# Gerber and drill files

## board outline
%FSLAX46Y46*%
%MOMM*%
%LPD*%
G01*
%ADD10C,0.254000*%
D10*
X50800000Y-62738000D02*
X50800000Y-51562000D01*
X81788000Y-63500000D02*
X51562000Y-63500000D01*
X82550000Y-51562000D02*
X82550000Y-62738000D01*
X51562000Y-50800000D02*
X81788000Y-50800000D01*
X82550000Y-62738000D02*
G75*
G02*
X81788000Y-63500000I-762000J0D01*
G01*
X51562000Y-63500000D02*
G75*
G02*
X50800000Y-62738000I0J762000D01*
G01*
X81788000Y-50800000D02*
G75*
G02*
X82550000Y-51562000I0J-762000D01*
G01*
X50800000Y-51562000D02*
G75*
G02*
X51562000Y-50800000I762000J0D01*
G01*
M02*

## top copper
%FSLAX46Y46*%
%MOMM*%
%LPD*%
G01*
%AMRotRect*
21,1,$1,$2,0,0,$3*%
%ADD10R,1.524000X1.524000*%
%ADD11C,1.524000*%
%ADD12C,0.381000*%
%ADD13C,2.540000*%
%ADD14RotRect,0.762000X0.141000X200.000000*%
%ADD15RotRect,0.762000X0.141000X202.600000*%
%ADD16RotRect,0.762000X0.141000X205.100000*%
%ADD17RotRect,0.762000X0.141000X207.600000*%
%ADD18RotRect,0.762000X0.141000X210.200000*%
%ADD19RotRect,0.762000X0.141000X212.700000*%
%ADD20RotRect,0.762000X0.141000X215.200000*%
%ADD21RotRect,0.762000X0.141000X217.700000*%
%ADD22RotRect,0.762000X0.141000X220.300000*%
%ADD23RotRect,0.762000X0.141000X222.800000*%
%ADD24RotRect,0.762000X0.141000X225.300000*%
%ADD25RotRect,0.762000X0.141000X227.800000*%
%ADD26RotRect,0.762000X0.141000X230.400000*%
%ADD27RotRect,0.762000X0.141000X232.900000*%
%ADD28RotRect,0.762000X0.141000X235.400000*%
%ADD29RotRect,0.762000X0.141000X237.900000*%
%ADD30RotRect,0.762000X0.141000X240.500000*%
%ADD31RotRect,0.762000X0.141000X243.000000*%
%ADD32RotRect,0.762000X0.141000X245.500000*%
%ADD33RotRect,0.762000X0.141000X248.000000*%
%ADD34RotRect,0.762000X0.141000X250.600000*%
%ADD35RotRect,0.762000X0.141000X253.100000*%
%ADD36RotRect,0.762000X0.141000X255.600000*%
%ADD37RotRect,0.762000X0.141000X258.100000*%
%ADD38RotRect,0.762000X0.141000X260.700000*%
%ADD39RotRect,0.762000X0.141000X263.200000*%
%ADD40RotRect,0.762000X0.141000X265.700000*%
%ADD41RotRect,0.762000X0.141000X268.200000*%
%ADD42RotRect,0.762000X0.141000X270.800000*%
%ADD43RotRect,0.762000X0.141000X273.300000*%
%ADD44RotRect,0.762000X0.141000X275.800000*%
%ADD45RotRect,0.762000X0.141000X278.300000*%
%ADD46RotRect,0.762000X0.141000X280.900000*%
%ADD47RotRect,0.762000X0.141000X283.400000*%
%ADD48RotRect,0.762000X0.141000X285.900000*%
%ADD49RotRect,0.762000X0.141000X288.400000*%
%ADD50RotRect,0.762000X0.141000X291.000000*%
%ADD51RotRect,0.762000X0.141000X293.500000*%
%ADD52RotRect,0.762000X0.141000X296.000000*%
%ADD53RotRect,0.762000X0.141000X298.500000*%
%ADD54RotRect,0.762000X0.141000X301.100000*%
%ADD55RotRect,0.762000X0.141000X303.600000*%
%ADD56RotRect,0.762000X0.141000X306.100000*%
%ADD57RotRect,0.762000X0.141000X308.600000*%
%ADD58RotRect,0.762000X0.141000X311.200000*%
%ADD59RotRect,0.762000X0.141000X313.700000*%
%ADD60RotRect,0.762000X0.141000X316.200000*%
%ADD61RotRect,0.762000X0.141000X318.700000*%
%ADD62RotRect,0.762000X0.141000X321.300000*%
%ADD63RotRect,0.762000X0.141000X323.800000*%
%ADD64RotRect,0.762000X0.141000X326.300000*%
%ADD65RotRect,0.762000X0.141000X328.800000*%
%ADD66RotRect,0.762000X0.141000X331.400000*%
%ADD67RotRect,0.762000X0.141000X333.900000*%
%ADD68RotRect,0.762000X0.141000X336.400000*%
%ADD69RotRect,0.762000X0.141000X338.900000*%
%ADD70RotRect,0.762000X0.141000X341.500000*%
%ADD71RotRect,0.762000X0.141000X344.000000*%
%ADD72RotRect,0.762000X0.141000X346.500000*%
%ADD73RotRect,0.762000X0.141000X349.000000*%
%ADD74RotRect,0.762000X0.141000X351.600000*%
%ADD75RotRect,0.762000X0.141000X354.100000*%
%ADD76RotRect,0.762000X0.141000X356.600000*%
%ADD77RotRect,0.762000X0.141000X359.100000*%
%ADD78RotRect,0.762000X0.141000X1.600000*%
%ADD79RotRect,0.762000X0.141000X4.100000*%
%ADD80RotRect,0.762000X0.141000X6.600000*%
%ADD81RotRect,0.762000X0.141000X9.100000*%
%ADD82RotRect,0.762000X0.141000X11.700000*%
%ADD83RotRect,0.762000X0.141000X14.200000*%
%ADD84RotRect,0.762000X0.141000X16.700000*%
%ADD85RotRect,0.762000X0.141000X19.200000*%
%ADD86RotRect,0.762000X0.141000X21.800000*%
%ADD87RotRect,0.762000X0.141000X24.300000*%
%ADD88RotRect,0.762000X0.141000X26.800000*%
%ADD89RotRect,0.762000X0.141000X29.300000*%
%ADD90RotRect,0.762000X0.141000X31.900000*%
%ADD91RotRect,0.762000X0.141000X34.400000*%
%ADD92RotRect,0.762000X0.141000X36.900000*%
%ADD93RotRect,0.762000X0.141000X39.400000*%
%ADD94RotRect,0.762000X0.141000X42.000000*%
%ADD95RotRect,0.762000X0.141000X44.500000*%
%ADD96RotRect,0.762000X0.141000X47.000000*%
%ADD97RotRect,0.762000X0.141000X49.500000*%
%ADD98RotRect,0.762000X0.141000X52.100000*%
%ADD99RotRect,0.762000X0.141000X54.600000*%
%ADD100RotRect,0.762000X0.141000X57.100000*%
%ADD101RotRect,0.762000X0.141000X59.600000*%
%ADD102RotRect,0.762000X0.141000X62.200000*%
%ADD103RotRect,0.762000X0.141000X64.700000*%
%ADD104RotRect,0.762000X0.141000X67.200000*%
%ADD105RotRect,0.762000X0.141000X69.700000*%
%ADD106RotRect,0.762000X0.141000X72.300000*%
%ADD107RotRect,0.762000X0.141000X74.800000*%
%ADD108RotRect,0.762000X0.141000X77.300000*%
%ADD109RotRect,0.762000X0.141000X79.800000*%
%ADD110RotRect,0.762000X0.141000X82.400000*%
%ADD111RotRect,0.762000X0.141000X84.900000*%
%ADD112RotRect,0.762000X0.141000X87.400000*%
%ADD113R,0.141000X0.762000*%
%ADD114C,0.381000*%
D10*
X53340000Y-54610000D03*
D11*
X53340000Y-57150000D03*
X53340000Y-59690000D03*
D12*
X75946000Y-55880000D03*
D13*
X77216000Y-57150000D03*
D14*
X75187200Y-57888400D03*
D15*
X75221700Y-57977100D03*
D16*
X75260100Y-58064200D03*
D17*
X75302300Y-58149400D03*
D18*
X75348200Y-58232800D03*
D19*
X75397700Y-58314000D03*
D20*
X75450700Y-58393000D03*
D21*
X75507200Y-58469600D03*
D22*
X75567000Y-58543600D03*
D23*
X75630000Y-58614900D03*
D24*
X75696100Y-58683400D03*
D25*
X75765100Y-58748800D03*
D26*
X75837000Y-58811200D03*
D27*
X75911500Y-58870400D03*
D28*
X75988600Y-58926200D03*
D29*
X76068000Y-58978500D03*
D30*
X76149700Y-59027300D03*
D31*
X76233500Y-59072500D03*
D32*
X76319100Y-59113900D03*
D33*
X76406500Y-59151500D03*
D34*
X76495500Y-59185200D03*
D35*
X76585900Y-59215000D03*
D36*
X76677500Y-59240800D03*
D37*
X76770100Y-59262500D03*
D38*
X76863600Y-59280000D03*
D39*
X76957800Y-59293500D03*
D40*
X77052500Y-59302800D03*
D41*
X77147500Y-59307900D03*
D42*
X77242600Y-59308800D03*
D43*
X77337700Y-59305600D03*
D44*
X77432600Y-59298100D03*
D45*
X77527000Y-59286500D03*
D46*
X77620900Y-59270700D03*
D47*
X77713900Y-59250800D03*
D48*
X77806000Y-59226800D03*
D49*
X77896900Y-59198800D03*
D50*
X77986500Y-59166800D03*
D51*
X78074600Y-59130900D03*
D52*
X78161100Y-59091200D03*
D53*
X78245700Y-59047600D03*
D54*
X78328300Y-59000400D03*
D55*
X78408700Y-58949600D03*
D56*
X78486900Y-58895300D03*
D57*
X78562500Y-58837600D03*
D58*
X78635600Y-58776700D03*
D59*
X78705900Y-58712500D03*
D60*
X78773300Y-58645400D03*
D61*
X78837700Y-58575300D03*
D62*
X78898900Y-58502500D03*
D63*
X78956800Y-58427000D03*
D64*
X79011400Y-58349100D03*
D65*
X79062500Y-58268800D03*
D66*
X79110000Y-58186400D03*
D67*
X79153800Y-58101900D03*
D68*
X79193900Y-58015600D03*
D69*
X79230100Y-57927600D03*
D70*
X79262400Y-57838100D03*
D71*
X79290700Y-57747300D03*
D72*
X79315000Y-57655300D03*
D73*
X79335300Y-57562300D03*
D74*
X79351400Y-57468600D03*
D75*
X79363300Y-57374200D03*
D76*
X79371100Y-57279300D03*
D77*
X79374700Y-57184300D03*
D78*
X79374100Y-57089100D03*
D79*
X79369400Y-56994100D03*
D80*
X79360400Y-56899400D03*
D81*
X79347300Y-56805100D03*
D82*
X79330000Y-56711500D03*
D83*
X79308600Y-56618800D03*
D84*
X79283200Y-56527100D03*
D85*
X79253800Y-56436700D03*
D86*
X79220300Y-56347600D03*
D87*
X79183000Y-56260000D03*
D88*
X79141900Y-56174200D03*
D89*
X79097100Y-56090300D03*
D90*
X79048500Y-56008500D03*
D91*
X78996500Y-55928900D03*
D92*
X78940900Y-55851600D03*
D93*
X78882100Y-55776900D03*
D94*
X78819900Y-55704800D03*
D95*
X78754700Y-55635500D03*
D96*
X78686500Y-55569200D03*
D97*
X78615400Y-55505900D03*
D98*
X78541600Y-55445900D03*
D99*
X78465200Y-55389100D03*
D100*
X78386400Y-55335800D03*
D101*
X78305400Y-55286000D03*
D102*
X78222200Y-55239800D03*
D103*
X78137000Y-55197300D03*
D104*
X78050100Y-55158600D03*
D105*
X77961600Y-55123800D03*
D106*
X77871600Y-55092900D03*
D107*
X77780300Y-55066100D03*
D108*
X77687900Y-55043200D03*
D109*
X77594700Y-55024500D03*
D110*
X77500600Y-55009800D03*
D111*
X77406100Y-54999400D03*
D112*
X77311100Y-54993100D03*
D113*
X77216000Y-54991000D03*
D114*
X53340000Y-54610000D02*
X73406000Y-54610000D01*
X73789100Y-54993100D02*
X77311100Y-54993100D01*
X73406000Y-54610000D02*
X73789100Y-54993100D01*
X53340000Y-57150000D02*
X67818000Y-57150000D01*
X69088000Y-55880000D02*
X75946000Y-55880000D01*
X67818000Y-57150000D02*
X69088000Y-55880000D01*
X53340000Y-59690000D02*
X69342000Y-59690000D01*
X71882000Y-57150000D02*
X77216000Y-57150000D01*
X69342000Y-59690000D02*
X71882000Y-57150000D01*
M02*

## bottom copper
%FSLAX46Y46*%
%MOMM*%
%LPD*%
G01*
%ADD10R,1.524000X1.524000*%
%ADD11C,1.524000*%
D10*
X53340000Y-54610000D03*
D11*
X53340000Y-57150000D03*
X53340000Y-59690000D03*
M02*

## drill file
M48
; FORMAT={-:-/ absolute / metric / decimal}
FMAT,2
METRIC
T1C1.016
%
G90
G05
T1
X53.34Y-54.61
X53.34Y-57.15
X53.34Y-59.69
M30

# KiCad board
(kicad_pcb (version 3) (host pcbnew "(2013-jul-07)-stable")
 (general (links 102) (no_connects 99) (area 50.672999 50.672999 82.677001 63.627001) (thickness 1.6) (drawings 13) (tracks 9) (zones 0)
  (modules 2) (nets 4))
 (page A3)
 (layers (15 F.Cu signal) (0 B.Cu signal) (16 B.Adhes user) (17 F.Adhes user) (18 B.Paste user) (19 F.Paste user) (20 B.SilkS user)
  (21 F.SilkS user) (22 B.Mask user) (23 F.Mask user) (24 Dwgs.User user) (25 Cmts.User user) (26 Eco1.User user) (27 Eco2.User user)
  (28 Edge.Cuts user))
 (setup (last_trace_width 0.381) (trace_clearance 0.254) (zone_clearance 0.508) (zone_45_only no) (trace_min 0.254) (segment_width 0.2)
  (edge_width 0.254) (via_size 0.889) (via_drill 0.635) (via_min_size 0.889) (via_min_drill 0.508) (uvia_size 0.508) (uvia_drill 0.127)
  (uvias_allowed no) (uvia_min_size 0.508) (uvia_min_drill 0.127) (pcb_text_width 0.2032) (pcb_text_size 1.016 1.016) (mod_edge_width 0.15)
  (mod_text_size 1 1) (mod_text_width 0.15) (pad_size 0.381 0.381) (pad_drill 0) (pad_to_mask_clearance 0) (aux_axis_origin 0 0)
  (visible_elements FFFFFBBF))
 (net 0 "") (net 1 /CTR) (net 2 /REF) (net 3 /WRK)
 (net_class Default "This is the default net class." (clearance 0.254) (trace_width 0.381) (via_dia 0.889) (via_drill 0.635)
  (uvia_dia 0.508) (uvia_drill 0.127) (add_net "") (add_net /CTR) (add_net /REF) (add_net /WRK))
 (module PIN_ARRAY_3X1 (layer F.Cu) (at 53.34 57.15 270)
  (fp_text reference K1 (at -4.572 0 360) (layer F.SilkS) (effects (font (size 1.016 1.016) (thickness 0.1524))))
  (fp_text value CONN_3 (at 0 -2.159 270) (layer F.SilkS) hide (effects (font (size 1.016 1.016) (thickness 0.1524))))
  (pad 1 thru_hole rect (at -2.54 0 270) (size 1.524 1.524) (drill 1.016) (layers *.Cu *.Mask F.SilkS) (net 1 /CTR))
  (pad 2 thru_hole circle (at 0 0 270) (size 1.524 1.524) (drill 1.016) (layers *.Cu *.Mask F.SilkS) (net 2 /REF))
  (pad 3 thru_hole circle (at 2.54 0 270) (size 1.524 1.524) (drill 1.016) (layers *.Cu *.Mask F.SilkS) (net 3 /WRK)))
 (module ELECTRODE (layer F.Cu) (at 77.216 57.15)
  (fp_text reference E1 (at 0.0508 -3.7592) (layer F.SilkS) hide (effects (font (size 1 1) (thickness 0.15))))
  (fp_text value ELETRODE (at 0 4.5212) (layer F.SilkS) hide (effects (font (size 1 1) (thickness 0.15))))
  (pad 1 smd circle (at -1.27 -1.27 225) (size 0.381 0.381) (layers F.Cu F.Paste F.Mask) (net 2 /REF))
  (pad 2 smd circle (at 0 0) (size 2.54 2.54) (layers F.Cu F.Paste F.Mask) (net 3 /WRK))
  (pad 3 smd rect (at -2.0288 0.7384 200) (size 0.762 0.141) (layers F.Cu F.Paste F.Mask) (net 1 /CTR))
  (pad 3 smd rect (at -1.9943 0.8271 202.6) (size 0.762 0.141) (layers F.Cu F.Paste F.Mask) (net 1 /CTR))
  (pad 3 smd rect (at -1.9559 0.9142 205.1) (size 0.762 0.141) (layers F.Cu F.Paste F.Mask) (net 1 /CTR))
  (pad 3 smd rect (at -1.9137 0.9994 207.6) (size 0.762 0.141) (layers F.Cu F.Paste F.Mask) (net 1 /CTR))
  (pad 3 smd rect (at -1.8678 1.0828 210.2) (size 0.762 0.141) (layers F.Cu F.Paste F.Mask) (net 1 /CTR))
  (pad 3 smd rect (at -1.8183 1.164 212.7) (size 0.762 0.141) (layers F.Cu F.Paste F.Mask) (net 1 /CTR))
  (pad 3 smd rect (at -1.7653 1.243 215.2) (size 0.762 0.141) (layers F.Cu F.Paste F.Mask) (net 1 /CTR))
  (pad 3 smd rect (at -1.7088 1.3196 217.7) (size 0.762 0.141) (layers F.Cu F.Paste F.Mask) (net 1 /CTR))
  (pad 3 smd rect (at -1.649 1.3936 220.3) (size 0.762 0.141) (layers F.Cu F.Paste F.Mask) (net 1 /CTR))
  (pad 3 smd rect (at -1.586 1.4649 222.8) (size 0.762 0.141) (layers F.Cu F.Paste F.Mask) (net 1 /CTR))
  (pad 3 smd rect (at -1.5199 1.5334 225.3) (size 0.762 0.141) (layers F.Cu F.Paste F.Mask) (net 1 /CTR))
  (pad 3 smd rect (at -1.4509 1.5988 227.8) (size 0.762 0.141) (layers F.Cu F.Paste F.Mask) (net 1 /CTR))
  (pad 3 smd rect (at -1.379 1.6612 230.4) (size 0.762 0.141) (layers F.Cu F.Paste F.Mask) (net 1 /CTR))
  (pad 3 smd rect (at -1.3045 1.7204 232.9) (size 0.762 0.141) (layers F.Cu F.Paste F.Mask) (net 1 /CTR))
  (pad 3 smd rect (at -1.2274 1.7762 235.4) (size 0.762 0.141) (layers F.Cu F.Paste F.Mask) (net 1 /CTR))
  (pad 3 smd rect (at -1.148 1.8285 237.9) (size 0.762 0.141) (layers F.Cu F.Paste F.Mask) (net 1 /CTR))
  (pad 3 smd rect (at -1.0663 1.8773 240.5) (size 0.762 0.141) (layers F.Cu F.Paste F.Mask) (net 1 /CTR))
  (pad 3 smd rect (at -0.9825 1.9225 243) (size 0.762 0.141) (layers F.Cu F.Paste F.Mask) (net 1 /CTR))
  (pad 3 smd rect (at -0.8969 1.9639 245.5) (size 0.762 0.141) (layers F.Cu F.Paste F.Mask) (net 1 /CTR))
  (pad 3 smd rect (at -0.8095 2.0015 248) (size 0.762 0.141) (layers F.Cu F.Paste F.Mask) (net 1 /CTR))
  (pad 3 smd rect (at -0.7205 2.0352 250.6) (size 0.762 0.141) (layers F.Cu F.Paste F.Mask) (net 1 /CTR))
  (pad 3 smd rect (at -0.6301 2.065 253.1) (size 0.762 0.141) (layers F.Cu F.Paste F.Mask) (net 1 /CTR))
  (pad 3 smd rect (at -0.5385 2.0908 255.6) (size 0.762 0.141) (layers F.Cu F.Paste F.Mask) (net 1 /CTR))
  (pad 3 smd rect (at -0.4459 2.1125 258.1) (size 0.762 0.141) (layers F.Cu F.Paste F.Mask) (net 1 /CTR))
  (pad 3 smd rect (at -0.3524 2.13 260.7) (size 0.762 0.141) (layers F.Cu F.Paste F.Mask) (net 1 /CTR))
  (pad 3 smd rect (at -0.2582 2.1435 263.2) (size 0.762 0.141) (layers F.Cu F.Paste F.Mask) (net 1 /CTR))
  (pad 3 smd rect (at -0.1635 2.1528 265.7) (size 0.762 0.141) (layers F.Cu F.Paste F.Mask) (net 1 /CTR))
  (pad 3 smd rect (at -0.0685 2.1579 268.2) (size 0.762 0.141) (layers F.Cu F.Paste F.Mask) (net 1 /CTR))
  (pad 3 smd rect (at 0.0266 2.1588 270.8) (size 0.762 0.141) (layers F.Cu F.Paste F.Mask) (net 1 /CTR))
  (pad 3 smd rect (at 0.1217 2.1556 273.3) (size 0.762 0.141) (layers F.Cu F.Paste F.Mask) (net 1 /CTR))
  (pad 3 smd rect (at 0.2166 2.1481 275.8) (size 0.762 0.141) (layers F.Cu F.Paste F.Mask) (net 1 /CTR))
  (pad 3 smd rect (at 0.311 2.1365 278.3) (size 0.762 0.141) (layers F.Cu F.Paste F.Mask) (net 1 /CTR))
  (pad 3 smd rect (at 0.4049 2.1207 280.9) (size 0.762 0.141) (layers F.Cu F.Paste F.Mask) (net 1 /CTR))
  (pad 3 smd rect (at 0.4979 2.1008 283.4) (size 0.762 0.141) (layers F.Cu F.Paste F.Mask) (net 1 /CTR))
  (pad 3 smd rect (at 0.59 2.0768 285.9) (size 0.762 0.141) (layers F.Cu F.Paste F.Mask) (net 1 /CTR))
  (pad 3 smd rect (at 0.6809 2.0488 288.4) (size 0.762 0.141) (layers F.Cu F.Paste F.Mask) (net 1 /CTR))
  (pad 3 smd rect (at 0.7705 2.0168 291) (size 0.762 0.141) (layers F.Cu F.Paste F.Mask) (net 1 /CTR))
  (pad 3 smd rect (at 0.8586 1.9809 293.5) (size 0.762 0.141) (layers F.Cu F.Paste F.Mask) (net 1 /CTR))
  (pad 3 smd rect (at 0.9451 1.9412 296) (size 0.762 0.141) (layers F.Cu F.Paste F.Mask) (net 1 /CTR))
  (pad 3 smd rect (at 1.0297 1.8976 298.5) (size 0.762 0.141) (layers F.Cu F.Paste F.Mask) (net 1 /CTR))
  (pad 3 smd rect (at 1.1123 1.8504 301.1) (size 0.762 0.141) (layers F.Cu F.Paste F.Mask) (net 1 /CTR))
  (pad 3 smd rect (at 1.1927 1.7996 303.6) (size 0.762 0.141) (layers F.Cu F.Paste F.Mask) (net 1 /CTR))
  (pad 3 smd rect (at 1.2709 1.7453 306.1) (size 0.762 0.141) (layers F.Cu F.Paste F.Mask) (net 1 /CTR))
  (pad 3 smd rect (at 1.3465 1.6876 308.6) (size 0.762 0.141) (layers F.Cu F.Paste F.Mask) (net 1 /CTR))
  (pad 3 smd rect (at 1.4196 1.6267 311.2) (size 0.762 0.141) (layers F.Cu F.Paste F.Mask) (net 1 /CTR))
  (pad 3 smd rect (at 1.4899 1.5625 313.7) (size 0.762 0.141) (layers F.Cu F.Paste F.Mask) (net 1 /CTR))
  (pad 3 smd rect (at 1.5573 1.4954 316.2) (size 0.762 0.141) (layers F.Cu F.Paste F.Mask) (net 1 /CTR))
  (pad 3 smd rect (at 1.6217 1.4253 318.7) (size 0.762 0.141) (layers F.Cu F.Paste F.Mask) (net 1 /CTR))
  (pad 3 smd rect (at 1.6829 1.3525 321.3) (size 0.762 0.141) (layers F.Cu F.Paste F.Mask) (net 1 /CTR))
  (pad 3 smd rect (at 1.7408 1.277 323.8) (size 0.762 0.141) (layers F.Cu F.Paste F.Mask) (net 1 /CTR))
  (pad 3 smd rect (at 1.7954 1.1991 326.3) (size 0.762 0.141) (layers F.Cu F.Paste F.Mask) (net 1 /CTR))
  (pad 3 smd rect (at 1.8465 1.1188 328.8) (size 0.762 0.141) (layers F.Cu F.Paste F.Mask) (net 1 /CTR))
  (pad 3 smd rect (at 1.894 1.0364 331.4) (size 0.762 0.141) (layers F.Cu F.Paste F.Mask) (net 1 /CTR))
  (pad 3 smd rect (at 1.9378 0.9519 333.9) (size 0.762 0.141) (layers F.Cu F.Paste F.Mask) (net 1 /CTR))
  (pad 3 smd rect (at 1.9779 0.8656 336.4) (size 0.762 0.141) (layers F.Cu F.Paste F.Mask) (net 1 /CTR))
  (pad 3 smd rect (at 2.0141 0.7776 338.9) (size 0.762 0.141) (layers F.Cu F.Paste F.Mask) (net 1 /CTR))
  (pad 3 smd rect (at 2.0464 0.6881 341.5) (size 0.762 0.141) (layers F.Cu F.Paste F.Mask) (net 1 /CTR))
  (pad 3 smd rect (at 2.0747 0.5973 344) (size 0.762 0.141) (layers F.Cu F.Paste F.Mask) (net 1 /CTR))
  (pad 3 smd rect (at 2.099 0.5053 346.5) (size 0.762 0.141) (layers F.Cu F.Paste F.Mask) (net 1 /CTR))
  (pad 3 smd rect (at 2.1193 0.4123 349) (size 0.762 0.141) (layers F.Cu F.Paste F.Mask) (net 1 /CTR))
  (pad 3 smd rect (at 2.1354 0.3186 351.6) (size 0.762 0.141) (layers F.Cu F.Paste F.Mask) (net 1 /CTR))
  (pad 3 smd rect (at 2.1473 0.2242 354.1) (size 0.762 0.141) (layers F.Cu F.Paste F.Mask) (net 1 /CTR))
  (pad 3 smd rect (at 2.1551 0.1293 356.6) (size 0.762 0.141) (layers F.Cu F.Paste F.Mask) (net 1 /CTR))
  (pad 3 smd rect (at 2.1587 0.0343 359.1) (size 0.762 0.141) (layers F.Cu F.Paste F.Mask) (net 1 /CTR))
  (pad 3 smd rect (at 2.1581 -0.0609 1.6) (size 0.762 0.141) (layers F.Cu F.Paste F.Mask) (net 1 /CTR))
  (pad 3 smd rect (at 2.1534 -0.1559 4.1) (size 0.762 0.141) (layers F.Cu F.Paste F.Mask) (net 1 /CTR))
  (pad 3 smd rect (at 2.1444 -0.2506 6.6) (size 0.762 0.141) (layers F.Cu F.Paste F.Mask) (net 1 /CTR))
  (pad 3 smd rect (at 2.1313 -0.3449 9.1) (size 0.762 0.141) (layers F.Cu F.Paste F.Mask) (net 1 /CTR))
  (pad 3 smd rect (at 2.114 -0.4385 11.7) (size 0.762 0.141) (layers F.Cu F.Paste F.Mask) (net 1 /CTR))
  (pad 3 smd rect (at 2.0926 -0.5312 14.2) (size 0.762 0.141) (layers F.Cu F.Paste F.Mask) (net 1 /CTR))
  (pad 3 smd rect (at 2.0672 -0.6229 16.7) (size 0.762 0.141) (layers F.Cu F.Paste F.Mask) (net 1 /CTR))
  (pad 3 smd rect (at 2.0378 -0.7133 19.2) (size 0.762 0.141) (layers F.Cu F.Paste F.Mask) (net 1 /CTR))
  (pad 3 smd rect (at 2.0043 -0.8024 21.8) (size 0.762 0.141) (layers F.Cu F.Paste F.Mask) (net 1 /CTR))
  (pad 3 smd rect (at 1.967 -0.89 24.3) (size 0.762 0.141) (layers F.Cu F.Paste F.Mask) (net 1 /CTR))
  (pad 3 smd rect (at 1.9259 -0.9758 26.8) (size 0.762 0.141) (layers F.Cu F.Paste F.Mask) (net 1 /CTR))
  (pad 3 smd rect (at 1.8811 -1.0597 29.3) (size 0.762 0.141) (layers F.Cu F.Paste F.Mask) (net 1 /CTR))
  (pad 3 smd rect (at 1.8325 -1.1415 31.9) (size 0.762 0.141) (layers F.Cu F.Paste F.Mask) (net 1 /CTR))
  (pad 3 smd rect (at 1.7805 -1.2211 34.4) (size 0.762 0.141) (layers F.Cu F.Paste F.Mask) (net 1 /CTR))
  (pad 3 smd rect (at 1.7249 -1.2984 36.9) (size 0.762 0.141) (layers F.Cu F.Paste F.Mask) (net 1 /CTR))
  (pad 3 smd rect (at 1.6661 -1.3731 39.4) (size 0.762 0.141) (layers F.Cu F.Paste F.Mask) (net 1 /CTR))
  (pad 3 smd rect (at 1.6039 -1.4452 42) (size 0.762 0.141) (layers F.Cu F.Paste F.Mask) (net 1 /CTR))
  (pad 3 smd rect (at 1.5387 -1.5145 44.5) (size 0.762 0.141) (layers F.Cu F.Paste F.Mask) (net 1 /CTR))
  (pad 3 smd rect (at 1.4705 -1.5808 47) (size 0.762 0.141) (layers F.Cu F.Paste F.Mask) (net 1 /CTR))
  (pad 3 smd rect (at 1.3994 -1.6441 49.5) (size 0.762 0.141) (layers F.Cu F.Paste F.Mask) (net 1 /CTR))
  (pad 3 smd rect (at 1.3256 -1.7041 52.1) (size 0.762 0.141) (layers F.Cu F.Paste F.Mask) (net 1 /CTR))
  (pad 3 smd rect (at 1.2492 -1.7609 54.6) (size 0.762 0.141) (layers F.Cu F.Paste F.Mask) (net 1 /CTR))
  (pad 3 smd rect (at 1.1704 -1.8142 57.1) (size 0.762 0.141) (layers F.Cu F.Paste F.Mask) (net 1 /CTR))
  (pad 3 smd rect (at 1.0894 -1.864 59.6) (size 0.762 0.141) (layers F.Cu F.Paste F.Mask) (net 1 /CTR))
  (pad 3 smd rect (at 1.0062 -1.9102 62.2) (size 0.762 0.141) (layers F.Cu F.Paste F.Mask) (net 1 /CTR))
  (pad 3 smd rect (at 0.921 -1.9527 64.7) (size 0.762 0.141) (layers F.Cu F.Paste F.Mask) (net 1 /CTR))
  (pad 3 smd rect (at 0.8341 -1.9914 67.2) (size 0.762 0.141) (layers F.Cu F.Paste F.Mask) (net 1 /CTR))
  (pad 3 smd rect (at 0.7456 -2.0262 69.7) (size 0.762 0.141) (layers F.Cu F.Paste F.Mask) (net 1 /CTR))
  (pad 3 smd rect (at 0.6556 -2.0571 72.3) (size 0.762 0.141) (layers F.Cu F.Paste F.Mask) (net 1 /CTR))
  (pad 3 smd rect (at 0.5643 -2.0839 74.8) (size 0.762 0.141) (layers F.Cu F.Paste F.Mask) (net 1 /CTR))
  (pad 3 smd rect (at 0.4719 -2.1068 77.3) (size 0.762 0.141) (layers F.Cu F.Paste F.Mask) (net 1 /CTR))
  (pad 3 smd rect (at 0.3787 -2.1255 79.8) (size 0.762 0.141) (layers F.Cu F.Paste F.Mask) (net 1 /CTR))
  (pad 3 smd rect (at 0.2846 -2.1402 82.4) (size 0.762 0.141) (layers F.Cu F.Paste F.Mask) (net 1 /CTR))
  (pad 3 smd rect (at 0.1901 -2.1506 84.9) (size 0.762 0.141) (layers F.Cu F.Paste F.Mask) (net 1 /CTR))
  (pad 3 smd rect (at 0.0951 -2.1569 87.4) (size 0.762 0.141) (layers F.Cu F.Paste F.Mask) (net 1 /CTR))
  (pad 3 smd rect (at 0 -2.159 90) (size 0.762 0.141) (layers F.Cu F.Paste F.Mask) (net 1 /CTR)))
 (gr_line (start 50.8 62.738) (end 50.8 51.562) (angle 90) (layer Edge.Cuts) (width 0.254))
 (gr_line (start 81.788 63.5) (end 51.562 63.5) (angle 90) (layer Edge.Cuts) (width 0.254))
 (gr_line (start 82.55 51.562) (end 82.55 62.738) (angle 90) (layer Edge.Cuts) (width 0.254))
 (gr_line (start 51.562 50.8) (end 81.788 50.8) (angle 90) (layer Edge.Cuts) (width 0.254))
 (gr_arc (start 81.788 62.738) (end 82.55 62.738) (angle 90) (layer Edge.Cuts) (width 0.254))
 (gr_arc (start 51.562 62.738) (end 51.562 63.5) (angle 90) (layer Edge.Cuts) (width 0.254))
 (gr_arc (start 81.788 51.562) (end 81.788 50.8) (angle 90) (layer Edge.Cuts) (width 0.254))
 (gr_arc (start 51.562 51.562) (end 50.8 51.562) (angle 90) (layer Edge.Cuts) (width 0.254))
 (segment (start 53.34 54.61) (end 73.406 54.61) (width 0.381) (layer F.Cu) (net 1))
 (segment (start 73.7891 54.9931) (end 77.3111 54.9931) (width 0.381) (layer F.Cu) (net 1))
 (segment (start 73.406 54.61) (end 73.7891 54.9931) (width 0.381) (layer F.Cu) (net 1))
 (segment (start 53.34 57.15) (end 67.818 57.15) (width 0.381) (layer F.Cu) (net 2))
 (segment (start 69.088 55.88) (end 75.946 55.88) (width 0.381) (layer F.Cu) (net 2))
 (segment (start 67.818 57.15) (end 69.088 55.88) (width 0.381) (layer F.Cu) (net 2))
 (segment (start 53.34 59.69) (end 69.342 59.69) (width 0.381) (layer F.Cu) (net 3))
 (segment (start 71.882 57.15) (end 77.216 57.15) (width 0.381) (layer F.Cu) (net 3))
 (segment (start 69.342 59.69) (end 71.882 57.15) (width 0.381) (layer F.Cu) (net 3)))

